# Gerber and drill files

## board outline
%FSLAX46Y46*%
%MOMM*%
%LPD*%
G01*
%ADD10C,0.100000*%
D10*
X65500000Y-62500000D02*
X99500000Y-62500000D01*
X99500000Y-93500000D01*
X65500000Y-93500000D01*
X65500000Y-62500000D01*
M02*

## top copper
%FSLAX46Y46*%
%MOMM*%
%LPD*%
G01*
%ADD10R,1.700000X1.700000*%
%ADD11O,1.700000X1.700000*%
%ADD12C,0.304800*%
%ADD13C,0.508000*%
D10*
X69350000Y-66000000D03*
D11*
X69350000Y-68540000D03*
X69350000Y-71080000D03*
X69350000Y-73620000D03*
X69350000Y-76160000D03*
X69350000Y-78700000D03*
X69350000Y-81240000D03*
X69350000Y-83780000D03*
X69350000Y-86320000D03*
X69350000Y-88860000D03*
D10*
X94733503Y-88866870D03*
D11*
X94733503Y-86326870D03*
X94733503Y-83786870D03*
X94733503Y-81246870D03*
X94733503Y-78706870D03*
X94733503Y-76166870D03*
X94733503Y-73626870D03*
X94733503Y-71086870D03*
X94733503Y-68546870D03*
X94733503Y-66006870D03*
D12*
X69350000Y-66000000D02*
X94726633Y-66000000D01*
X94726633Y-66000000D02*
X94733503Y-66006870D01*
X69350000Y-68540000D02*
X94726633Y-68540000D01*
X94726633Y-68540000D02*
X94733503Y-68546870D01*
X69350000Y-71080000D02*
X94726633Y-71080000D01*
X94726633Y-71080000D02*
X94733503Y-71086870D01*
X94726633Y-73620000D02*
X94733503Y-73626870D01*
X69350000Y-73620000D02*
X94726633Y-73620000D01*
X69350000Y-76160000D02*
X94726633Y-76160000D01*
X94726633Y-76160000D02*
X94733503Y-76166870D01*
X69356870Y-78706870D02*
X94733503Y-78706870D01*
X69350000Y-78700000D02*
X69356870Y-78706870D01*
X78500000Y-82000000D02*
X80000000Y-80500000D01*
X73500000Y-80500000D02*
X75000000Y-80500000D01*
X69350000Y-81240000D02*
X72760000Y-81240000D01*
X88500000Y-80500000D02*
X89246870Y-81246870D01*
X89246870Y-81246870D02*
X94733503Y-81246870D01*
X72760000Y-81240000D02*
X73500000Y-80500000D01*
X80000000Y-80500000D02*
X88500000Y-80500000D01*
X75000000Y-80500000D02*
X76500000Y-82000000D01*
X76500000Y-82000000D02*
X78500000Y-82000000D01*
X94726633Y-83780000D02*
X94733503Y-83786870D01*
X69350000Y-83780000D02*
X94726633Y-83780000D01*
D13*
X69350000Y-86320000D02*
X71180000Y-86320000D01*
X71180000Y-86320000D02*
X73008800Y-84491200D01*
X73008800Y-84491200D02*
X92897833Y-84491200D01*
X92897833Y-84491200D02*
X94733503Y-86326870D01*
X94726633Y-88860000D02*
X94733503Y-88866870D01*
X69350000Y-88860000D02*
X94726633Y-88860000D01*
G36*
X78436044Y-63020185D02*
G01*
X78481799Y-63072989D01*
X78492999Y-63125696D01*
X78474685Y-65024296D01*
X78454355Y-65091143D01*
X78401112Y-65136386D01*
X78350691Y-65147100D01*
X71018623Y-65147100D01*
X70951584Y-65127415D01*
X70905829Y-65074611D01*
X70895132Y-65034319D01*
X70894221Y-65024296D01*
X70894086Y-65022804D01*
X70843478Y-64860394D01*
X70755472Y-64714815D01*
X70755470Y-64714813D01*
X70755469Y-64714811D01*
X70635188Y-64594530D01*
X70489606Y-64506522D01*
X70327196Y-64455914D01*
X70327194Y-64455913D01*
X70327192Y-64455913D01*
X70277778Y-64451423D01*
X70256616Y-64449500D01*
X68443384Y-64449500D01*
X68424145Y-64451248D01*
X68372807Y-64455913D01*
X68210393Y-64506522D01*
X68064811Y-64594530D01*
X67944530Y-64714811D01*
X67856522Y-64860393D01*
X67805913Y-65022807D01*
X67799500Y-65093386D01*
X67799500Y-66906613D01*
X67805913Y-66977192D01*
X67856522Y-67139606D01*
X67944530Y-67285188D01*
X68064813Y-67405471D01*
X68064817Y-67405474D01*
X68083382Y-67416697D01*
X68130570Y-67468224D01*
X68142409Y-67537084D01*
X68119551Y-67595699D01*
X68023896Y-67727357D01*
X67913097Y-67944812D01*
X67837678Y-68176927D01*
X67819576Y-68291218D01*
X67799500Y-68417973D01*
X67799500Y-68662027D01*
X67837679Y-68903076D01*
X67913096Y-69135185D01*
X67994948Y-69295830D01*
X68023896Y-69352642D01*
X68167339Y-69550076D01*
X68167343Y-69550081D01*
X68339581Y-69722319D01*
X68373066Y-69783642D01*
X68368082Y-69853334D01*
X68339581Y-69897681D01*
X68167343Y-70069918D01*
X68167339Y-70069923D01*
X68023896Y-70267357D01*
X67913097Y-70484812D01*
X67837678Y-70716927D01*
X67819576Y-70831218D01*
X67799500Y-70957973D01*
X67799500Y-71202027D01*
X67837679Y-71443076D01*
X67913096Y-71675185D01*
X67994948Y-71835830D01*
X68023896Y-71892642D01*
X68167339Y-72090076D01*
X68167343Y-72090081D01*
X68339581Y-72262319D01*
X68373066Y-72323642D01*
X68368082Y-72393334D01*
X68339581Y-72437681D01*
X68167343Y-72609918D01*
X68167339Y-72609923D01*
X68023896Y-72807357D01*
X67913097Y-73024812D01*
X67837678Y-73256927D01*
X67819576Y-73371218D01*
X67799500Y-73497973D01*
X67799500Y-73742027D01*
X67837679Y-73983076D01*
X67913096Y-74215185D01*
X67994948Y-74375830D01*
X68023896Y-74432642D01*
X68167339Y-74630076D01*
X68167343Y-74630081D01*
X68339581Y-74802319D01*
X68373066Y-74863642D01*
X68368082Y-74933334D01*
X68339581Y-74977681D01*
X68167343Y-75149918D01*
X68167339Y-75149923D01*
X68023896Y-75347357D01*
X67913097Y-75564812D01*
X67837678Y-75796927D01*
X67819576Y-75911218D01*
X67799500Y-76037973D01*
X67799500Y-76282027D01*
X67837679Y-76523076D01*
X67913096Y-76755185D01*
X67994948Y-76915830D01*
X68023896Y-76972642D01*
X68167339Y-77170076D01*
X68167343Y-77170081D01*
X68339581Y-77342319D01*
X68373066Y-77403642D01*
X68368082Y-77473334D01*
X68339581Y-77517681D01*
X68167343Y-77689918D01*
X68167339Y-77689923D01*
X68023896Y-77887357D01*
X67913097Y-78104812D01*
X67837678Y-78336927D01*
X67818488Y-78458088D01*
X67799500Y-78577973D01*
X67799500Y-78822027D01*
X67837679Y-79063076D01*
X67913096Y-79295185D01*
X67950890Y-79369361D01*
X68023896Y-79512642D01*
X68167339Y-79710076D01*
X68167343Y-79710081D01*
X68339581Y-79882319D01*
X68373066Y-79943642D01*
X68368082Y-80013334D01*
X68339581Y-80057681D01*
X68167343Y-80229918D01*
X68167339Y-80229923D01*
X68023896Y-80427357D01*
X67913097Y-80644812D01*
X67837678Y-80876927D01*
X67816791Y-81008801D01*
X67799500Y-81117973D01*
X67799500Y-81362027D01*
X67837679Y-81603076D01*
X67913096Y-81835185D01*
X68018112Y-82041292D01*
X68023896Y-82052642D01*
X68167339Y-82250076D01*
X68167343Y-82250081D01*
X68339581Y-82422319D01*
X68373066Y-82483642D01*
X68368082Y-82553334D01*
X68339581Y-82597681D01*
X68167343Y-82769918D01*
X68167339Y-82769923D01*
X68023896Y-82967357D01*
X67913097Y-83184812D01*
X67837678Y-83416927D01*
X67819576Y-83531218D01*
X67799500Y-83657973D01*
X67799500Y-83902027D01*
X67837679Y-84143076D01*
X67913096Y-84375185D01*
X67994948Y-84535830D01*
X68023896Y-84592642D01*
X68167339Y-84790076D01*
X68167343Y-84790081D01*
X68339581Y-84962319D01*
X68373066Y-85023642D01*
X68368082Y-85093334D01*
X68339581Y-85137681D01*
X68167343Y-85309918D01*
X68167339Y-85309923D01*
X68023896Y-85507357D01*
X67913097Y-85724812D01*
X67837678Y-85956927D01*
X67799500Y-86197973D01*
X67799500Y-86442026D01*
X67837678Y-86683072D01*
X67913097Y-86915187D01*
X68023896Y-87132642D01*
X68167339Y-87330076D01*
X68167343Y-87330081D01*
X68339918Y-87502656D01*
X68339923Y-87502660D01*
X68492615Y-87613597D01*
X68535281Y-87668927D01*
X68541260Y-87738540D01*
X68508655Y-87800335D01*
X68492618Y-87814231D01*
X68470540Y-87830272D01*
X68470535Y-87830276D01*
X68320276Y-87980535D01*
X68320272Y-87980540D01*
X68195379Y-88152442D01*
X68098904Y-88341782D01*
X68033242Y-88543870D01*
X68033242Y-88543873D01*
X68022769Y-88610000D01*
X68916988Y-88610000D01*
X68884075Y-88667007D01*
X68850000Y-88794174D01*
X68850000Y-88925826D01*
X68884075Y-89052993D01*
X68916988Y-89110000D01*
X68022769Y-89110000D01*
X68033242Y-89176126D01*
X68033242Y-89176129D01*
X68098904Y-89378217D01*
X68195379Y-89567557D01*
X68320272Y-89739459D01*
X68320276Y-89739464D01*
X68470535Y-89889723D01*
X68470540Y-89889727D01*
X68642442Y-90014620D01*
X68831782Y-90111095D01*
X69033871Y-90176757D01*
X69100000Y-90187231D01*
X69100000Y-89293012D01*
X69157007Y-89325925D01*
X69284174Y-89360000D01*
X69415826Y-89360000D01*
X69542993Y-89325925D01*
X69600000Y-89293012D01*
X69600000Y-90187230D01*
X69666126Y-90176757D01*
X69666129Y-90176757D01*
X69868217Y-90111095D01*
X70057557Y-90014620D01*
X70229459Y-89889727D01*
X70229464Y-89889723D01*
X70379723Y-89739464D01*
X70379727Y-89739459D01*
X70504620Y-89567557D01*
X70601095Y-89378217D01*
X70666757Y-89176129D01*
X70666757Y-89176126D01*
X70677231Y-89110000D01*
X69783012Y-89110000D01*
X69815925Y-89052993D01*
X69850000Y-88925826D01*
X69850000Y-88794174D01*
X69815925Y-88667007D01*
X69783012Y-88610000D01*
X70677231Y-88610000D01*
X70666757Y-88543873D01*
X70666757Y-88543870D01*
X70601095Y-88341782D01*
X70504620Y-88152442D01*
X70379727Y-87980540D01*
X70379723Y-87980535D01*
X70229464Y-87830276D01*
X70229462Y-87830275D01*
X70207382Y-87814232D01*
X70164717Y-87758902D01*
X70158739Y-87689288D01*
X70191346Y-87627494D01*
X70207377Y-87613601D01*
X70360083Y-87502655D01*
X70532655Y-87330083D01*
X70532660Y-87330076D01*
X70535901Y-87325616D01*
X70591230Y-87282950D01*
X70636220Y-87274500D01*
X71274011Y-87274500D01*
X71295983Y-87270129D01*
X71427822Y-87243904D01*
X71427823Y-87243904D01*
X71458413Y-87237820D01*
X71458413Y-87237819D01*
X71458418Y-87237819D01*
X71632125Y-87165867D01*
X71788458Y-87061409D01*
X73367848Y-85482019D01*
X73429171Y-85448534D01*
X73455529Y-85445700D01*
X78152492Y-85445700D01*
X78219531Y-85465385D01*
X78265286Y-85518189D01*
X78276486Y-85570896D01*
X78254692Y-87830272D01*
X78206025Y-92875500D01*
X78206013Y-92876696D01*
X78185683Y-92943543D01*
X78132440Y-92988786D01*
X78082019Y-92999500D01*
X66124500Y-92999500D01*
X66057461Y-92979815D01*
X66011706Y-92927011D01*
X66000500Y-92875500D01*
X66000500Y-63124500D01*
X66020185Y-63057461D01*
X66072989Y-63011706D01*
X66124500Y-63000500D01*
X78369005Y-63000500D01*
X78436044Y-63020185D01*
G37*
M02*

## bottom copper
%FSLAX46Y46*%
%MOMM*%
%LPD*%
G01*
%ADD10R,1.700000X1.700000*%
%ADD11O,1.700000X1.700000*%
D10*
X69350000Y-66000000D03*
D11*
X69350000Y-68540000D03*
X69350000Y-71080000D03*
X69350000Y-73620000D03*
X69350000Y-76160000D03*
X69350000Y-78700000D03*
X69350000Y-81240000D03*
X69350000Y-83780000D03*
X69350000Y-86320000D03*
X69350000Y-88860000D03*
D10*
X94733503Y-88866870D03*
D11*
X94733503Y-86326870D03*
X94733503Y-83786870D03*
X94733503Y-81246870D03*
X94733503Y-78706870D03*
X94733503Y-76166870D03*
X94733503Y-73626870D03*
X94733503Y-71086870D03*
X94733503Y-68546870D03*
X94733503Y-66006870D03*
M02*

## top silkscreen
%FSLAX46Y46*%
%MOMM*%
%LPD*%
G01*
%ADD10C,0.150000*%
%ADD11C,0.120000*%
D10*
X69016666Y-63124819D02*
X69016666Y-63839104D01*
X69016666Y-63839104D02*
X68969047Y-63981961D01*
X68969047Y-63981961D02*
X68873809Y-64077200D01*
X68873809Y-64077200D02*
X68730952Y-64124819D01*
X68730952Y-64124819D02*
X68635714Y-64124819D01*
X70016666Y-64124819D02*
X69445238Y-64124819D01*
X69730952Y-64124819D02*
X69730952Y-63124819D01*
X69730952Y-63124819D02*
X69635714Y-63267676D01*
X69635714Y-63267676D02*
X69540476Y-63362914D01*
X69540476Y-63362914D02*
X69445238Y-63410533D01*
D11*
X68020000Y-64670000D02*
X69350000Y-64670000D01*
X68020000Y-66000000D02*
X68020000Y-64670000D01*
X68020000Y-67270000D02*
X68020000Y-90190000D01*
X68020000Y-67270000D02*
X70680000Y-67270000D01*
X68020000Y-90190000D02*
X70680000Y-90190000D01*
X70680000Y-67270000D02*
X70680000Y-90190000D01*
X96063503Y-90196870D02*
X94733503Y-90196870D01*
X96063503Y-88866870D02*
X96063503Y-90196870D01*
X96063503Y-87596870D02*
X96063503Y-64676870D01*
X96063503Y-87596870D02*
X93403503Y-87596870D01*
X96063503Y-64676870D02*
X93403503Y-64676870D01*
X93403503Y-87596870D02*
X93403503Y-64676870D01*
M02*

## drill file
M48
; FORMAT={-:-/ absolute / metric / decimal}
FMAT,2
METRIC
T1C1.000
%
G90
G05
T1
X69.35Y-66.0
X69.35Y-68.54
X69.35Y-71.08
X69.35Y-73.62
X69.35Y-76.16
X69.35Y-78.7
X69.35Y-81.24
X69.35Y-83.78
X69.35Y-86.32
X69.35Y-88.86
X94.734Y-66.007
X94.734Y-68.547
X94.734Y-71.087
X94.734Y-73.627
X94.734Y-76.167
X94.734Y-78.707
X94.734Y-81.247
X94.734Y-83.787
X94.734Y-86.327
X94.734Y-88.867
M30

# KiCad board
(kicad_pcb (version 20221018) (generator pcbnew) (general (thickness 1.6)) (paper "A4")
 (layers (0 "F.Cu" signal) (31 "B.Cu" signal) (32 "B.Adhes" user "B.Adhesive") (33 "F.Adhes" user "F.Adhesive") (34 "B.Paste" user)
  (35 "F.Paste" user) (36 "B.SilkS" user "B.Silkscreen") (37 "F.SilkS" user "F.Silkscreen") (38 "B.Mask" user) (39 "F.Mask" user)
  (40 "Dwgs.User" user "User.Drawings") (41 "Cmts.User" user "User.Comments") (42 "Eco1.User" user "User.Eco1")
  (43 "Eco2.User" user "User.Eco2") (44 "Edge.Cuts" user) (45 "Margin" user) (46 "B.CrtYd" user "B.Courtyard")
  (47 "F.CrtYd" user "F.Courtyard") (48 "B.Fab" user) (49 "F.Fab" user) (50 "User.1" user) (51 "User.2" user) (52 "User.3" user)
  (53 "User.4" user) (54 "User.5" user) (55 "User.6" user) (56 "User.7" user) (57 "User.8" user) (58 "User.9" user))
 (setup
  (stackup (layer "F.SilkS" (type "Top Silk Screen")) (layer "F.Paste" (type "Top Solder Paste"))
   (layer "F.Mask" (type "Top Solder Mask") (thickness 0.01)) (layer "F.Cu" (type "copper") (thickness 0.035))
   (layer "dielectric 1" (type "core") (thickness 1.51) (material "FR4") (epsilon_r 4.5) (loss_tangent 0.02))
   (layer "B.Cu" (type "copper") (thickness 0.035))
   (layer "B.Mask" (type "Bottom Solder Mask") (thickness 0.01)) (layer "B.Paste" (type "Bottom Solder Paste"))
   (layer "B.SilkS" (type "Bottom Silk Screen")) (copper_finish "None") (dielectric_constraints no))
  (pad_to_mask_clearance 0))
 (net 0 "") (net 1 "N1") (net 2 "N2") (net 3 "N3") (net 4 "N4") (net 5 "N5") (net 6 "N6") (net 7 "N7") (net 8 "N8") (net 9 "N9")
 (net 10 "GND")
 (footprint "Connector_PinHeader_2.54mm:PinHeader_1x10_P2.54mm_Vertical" (layer "F.Cu") (at 69.35 66)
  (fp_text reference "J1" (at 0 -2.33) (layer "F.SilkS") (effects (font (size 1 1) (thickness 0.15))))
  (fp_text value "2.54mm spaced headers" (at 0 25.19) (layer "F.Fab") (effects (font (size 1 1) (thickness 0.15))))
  (fp_line (start -1.33 -1.33) (end 0 -1.33) (stroke (width 0.12) (type solid)) (layer "F.SilkS"))
  (fp_line (start -1.33 0) (end -1.33 -1.33) (stroke (width 0.12) (type solid)) (layer "F.SilkS"))
  (fp_line (start -1.33 1.27) (end -1.33 24.19) (stroke (width 0.12) (type solid)) (layer "F.SilkS"))
  (fp_line (start -1.33 1.27) (end 1.33 1.27) (stroke (width 0.12) (type solid)) (layer "F.SilkS"))
  (fp_line (start -1.33 24.19) (end 1.33 24.19) (stroke (width 0.12) (type solid)) (layer "F.SilkS"))
  (fp_line (start 1.33 1.27) (end 1.33 24.19) (stroke (width 0.12) (type solid)) (layer "F.SilkS"))
  (pad "1" thru_hole rect (at 0 0) (size 1.7 1.7) (drill 1) (layers "*.Cu" "*.Mask") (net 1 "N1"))
  (pad "2" thru_hole oval (at 0 2.54) (size 1.7 1.7) (drill 1) (layers "*.Cu" "*.Mask") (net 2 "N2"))
  (pad "3" thru_hole oval (at 0 5.08) (size 1.7 1.7) (drill 1) (layers "*.Cu" "*.Mask") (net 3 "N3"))
  (pad "4" thru_hole oval (at 0 7.62) (size 1.7 1.7) (drill 1) (layers "*.Cu" "*.Mask") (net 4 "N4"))
  (pad "5" thru_hole oval (at 0 10.16) (size 1.7 1.7) (drill 1) (layers "*.Cu" "*.Mask") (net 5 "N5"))
  (pad "6" thru_hole oval (at 0 12.7) (size 1.7 1.7) (drill 1) (layers "*.Cu" "*.Mask") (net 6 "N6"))
  (pad "7" thru_hole oval (at 0 15.24) (size 1.7 1.7) (drill 1) (layers "*.Cu" "*.Mask") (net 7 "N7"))
  (pad "8" thru_hole oval (at 0 17.78) (size 1.7 1.7) (drill 1) (layers "*.Cu" "*.Mask") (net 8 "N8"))
  (pad "9" thru_hole oval (at 0 20.32) (size 1.7 1.7) (drill 1) (layers "*.Cu" "*.Mask") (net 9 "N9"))
  (pad "10" thru_hole oval (at 0 22.86) (size 1.7 1.7) (drill 1) (layers "*.Cu" "*.Mask") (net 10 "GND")))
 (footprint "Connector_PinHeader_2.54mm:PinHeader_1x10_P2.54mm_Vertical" (layer "F.Cu") (at 94.733503 88.86687 180)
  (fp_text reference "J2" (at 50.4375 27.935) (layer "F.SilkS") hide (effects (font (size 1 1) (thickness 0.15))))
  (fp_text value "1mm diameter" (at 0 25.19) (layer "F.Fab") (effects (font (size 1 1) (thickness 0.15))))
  (fp_line (start -1.33 -1.33) (end 0 -1.33) (stroke (width 0.12) (type solid)) (layer "F.SilkS"))
  (fp_line (start -1.33 0) (end -1.33 -1.33) (stroke (width 0.12) (type solid)) (layer "F.SilkS"))
  (fp_line (start -1.33 1.27) (end -1.33 24.19) (stroke (width 0.12) (type solid)) (layer "F.SilkS"))
  (fp_line (start -1.33 1.27) (end 1.33 1.27) (stroke (width 0.12) (type solid)) (layer "F.SilkS"))
  (fp_line (start -1.33 24.19) (end 1.33 24.19) (stroke (width 0.12) (type solid)) (layer "F.SilkS"))
  (fp_line (start 1.33 1.27) (end 1.33 24.19) (stroke (width 0.12) (type solid)) (layer "F.SilkS"))
  (pad "1" thru_hole rect (at 0 0 180) (size 1.7 1.7) (drill 1) (layers "*.Cu" "*.Mask") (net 10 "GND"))
  (pad "2" thru_hole oval (at 0 2.54 180) (size 1.7 1.7) (drill 1) (layers "*.Cu" "*.Mask") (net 9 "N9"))
  (pad "3" thru_hole oval (at 0 5.08 180) (size 1.7 1.7) (drill 1) (layers "*.Cu" "*.Mask") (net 8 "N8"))
  (pad "4" thru_hole oval (at 0 7.62 180) (size 1.7 1.7) (drill 1) (layers "*.Cu" "*.Mask") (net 7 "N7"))
  (pad "5" thru_hole oval (at 0 10.16 180) (size 1.7 1.7) (drill 1) (layers "*.Cu" "*.Mask") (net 6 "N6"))
  (pad "6" thru_hole oval (at 0 12.7 180) (size 1.7 1.7) (drill 1) (layers "*.Cu" "*.Mask") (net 5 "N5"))
  (pad "7" thru_hole oval (at 0 15.24 180) (size 1.7 1.7) (drill 1) (layers "*.Cu" "*.Mask") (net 4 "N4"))
  (pad "8" thru_hole oval (at 0 17.78 180) (size 1.7 1.7) (drill 1) (layers "*.Cu" "*.Mask") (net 3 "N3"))
  (pad "9" thru_hole oval (at 0 20.32 180) (size 1.7 1.7) (drill 1) (layers "*.Cu" "*.Mask") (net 2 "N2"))
  (pad "10" thru_hole oval (at 0 22.86 180) (size 1.7 1.7) (drill 1) (layers "*.Cu" "*.Mask") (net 1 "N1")))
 (gr_rect (start 65.5 62.5) (end 99.5 93.5) (stroke (width 0.1) (type default)) (fill none) (layer "Edge.Cuts"))
 (segment (start 69.35 66) (end 94.726633 66) (width 0.3048) (layer "F.Cu") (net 1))
 (segment (start 94.726633 66) (end 94.733503 66.00687) (width 0.3048) (layer "F.Cu") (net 1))
 (segment (start 69.35 68.54) (end 94.726633 68.54) (width 0.3048) (layer "F.Cu") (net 2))
 (segment (start 94.726633 68.54) (end 94.733503 68.54687) (width 0.3048) (layer "F.Cu") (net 2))
 (segment (start 69.35 71.08) (end 94.726633 71.08) (width 0.3048) (layer "F.Cu") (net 3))
 (segment (start 94.726633 71.08) (end 94.733503 71.08687) (width 0.3048) (layer "F.Cu") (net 3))
 (segment (start 94.726633 73.62) (end 94.733503 73.62687) (width 0.3048) (layer "F.Cu") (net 4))
 (segment (start 69.35 73.62) (end 94.726633 73.62) (width 0.3048) (layer "F.Cu") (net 4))
 (segment (start 69.35 76.16) (end 94.726633 76.16) (width 0.3048) (layer "F.Cu") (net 5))
 (segment (start 94.726633 76.16) (end 94.733503 76.16687) (width 0.3048) (layer "F.Cu") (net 5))
 (segment (start 69.35687 78.70687) (end 94.733503 78.70687) (width 0.3048) (layer "F.Cu") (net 6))
 (segment (start 69.35 78.7) (end 69.35687 78.70687) (width 0.3048) (layer "F.Cu") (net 6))
 (segment (start 78.5 82) (end 80 80.5) (width 0.3048) (layer "F.Cu") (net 7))
 (segment (start 73.5 80.5) (end 75 80.5) (width 0.3048) (layer "F.Cu") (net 7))
 (segment (start 69.35 81.24) (end 72.76 81.24) (width 0.3048) (layer "F.Cu") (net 7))
 (segment (start 88.5 80.5) (end 89.24687 81.24687) (width 0.3048) (layer "F.Cu") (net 7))
 (segment (start 89.24687 81.24687) (end 94.733503 81.24687) (width 0.3048) (layer "F.Cu") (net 7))
 (segment (start 72.76 81.24) (end 73.5 80.5) (width 0.3048) (layer "F.Cu") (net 7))
 (segment (start 80 80.5) (end 88.5 80.5) (width 0.3048) (layer "F.Cu") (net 7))
 (segment (start 75 80.5) (end 76.5 82) (width 0.3048) (layer "F.Cu") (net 7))
 (segment (start 76.5 82) (end 78.5 82) (width 0.3048) (layer "F.Cu") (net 7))
 (segment (start 94.726633 83.78) (end 94.733503 83.78687) (width 0.3048) (layer "F.Cu") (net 8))
 (segment (start 69.35 83.78) (end 94.726633 83.78) (width 0.3048) (layer "F.Cu") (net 8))
 (segment (start 69.35 86.32) (end 71.18 86.32) (width 0.508) (layer "F.Cu") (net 9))
 (segment (start 71.18 86.32) (end 73.0088 84.4912) (width 0.508) (layer "F.Cu") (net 9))
 (segment (start 73.0088 84.4912) (end 92.897833 84.4912) (width 0.508) (layer "F.Cu") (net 9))
 (segment (start 92.897833 84.4912) (end 94.733503 86.32687) (width 0.508) (layer "F.Cu") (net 9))
 (segment (start 94.726633 88.86) (end 94.733503 88.86687) (width 0.508) (layer "F.Cu") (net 10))
 (segment (start 69.35 88.86) (end 94.726633 88.86) (width 0.508) (layer "F.Cu") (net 10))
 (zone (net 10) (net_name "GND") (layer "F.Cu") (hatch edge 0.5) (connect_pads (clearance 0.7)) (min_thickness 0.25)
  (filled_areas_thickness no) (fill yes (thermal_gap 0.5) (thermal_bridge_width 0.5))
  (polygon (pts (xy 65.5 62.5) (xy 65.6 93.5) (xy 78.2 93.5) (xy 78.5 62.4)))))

